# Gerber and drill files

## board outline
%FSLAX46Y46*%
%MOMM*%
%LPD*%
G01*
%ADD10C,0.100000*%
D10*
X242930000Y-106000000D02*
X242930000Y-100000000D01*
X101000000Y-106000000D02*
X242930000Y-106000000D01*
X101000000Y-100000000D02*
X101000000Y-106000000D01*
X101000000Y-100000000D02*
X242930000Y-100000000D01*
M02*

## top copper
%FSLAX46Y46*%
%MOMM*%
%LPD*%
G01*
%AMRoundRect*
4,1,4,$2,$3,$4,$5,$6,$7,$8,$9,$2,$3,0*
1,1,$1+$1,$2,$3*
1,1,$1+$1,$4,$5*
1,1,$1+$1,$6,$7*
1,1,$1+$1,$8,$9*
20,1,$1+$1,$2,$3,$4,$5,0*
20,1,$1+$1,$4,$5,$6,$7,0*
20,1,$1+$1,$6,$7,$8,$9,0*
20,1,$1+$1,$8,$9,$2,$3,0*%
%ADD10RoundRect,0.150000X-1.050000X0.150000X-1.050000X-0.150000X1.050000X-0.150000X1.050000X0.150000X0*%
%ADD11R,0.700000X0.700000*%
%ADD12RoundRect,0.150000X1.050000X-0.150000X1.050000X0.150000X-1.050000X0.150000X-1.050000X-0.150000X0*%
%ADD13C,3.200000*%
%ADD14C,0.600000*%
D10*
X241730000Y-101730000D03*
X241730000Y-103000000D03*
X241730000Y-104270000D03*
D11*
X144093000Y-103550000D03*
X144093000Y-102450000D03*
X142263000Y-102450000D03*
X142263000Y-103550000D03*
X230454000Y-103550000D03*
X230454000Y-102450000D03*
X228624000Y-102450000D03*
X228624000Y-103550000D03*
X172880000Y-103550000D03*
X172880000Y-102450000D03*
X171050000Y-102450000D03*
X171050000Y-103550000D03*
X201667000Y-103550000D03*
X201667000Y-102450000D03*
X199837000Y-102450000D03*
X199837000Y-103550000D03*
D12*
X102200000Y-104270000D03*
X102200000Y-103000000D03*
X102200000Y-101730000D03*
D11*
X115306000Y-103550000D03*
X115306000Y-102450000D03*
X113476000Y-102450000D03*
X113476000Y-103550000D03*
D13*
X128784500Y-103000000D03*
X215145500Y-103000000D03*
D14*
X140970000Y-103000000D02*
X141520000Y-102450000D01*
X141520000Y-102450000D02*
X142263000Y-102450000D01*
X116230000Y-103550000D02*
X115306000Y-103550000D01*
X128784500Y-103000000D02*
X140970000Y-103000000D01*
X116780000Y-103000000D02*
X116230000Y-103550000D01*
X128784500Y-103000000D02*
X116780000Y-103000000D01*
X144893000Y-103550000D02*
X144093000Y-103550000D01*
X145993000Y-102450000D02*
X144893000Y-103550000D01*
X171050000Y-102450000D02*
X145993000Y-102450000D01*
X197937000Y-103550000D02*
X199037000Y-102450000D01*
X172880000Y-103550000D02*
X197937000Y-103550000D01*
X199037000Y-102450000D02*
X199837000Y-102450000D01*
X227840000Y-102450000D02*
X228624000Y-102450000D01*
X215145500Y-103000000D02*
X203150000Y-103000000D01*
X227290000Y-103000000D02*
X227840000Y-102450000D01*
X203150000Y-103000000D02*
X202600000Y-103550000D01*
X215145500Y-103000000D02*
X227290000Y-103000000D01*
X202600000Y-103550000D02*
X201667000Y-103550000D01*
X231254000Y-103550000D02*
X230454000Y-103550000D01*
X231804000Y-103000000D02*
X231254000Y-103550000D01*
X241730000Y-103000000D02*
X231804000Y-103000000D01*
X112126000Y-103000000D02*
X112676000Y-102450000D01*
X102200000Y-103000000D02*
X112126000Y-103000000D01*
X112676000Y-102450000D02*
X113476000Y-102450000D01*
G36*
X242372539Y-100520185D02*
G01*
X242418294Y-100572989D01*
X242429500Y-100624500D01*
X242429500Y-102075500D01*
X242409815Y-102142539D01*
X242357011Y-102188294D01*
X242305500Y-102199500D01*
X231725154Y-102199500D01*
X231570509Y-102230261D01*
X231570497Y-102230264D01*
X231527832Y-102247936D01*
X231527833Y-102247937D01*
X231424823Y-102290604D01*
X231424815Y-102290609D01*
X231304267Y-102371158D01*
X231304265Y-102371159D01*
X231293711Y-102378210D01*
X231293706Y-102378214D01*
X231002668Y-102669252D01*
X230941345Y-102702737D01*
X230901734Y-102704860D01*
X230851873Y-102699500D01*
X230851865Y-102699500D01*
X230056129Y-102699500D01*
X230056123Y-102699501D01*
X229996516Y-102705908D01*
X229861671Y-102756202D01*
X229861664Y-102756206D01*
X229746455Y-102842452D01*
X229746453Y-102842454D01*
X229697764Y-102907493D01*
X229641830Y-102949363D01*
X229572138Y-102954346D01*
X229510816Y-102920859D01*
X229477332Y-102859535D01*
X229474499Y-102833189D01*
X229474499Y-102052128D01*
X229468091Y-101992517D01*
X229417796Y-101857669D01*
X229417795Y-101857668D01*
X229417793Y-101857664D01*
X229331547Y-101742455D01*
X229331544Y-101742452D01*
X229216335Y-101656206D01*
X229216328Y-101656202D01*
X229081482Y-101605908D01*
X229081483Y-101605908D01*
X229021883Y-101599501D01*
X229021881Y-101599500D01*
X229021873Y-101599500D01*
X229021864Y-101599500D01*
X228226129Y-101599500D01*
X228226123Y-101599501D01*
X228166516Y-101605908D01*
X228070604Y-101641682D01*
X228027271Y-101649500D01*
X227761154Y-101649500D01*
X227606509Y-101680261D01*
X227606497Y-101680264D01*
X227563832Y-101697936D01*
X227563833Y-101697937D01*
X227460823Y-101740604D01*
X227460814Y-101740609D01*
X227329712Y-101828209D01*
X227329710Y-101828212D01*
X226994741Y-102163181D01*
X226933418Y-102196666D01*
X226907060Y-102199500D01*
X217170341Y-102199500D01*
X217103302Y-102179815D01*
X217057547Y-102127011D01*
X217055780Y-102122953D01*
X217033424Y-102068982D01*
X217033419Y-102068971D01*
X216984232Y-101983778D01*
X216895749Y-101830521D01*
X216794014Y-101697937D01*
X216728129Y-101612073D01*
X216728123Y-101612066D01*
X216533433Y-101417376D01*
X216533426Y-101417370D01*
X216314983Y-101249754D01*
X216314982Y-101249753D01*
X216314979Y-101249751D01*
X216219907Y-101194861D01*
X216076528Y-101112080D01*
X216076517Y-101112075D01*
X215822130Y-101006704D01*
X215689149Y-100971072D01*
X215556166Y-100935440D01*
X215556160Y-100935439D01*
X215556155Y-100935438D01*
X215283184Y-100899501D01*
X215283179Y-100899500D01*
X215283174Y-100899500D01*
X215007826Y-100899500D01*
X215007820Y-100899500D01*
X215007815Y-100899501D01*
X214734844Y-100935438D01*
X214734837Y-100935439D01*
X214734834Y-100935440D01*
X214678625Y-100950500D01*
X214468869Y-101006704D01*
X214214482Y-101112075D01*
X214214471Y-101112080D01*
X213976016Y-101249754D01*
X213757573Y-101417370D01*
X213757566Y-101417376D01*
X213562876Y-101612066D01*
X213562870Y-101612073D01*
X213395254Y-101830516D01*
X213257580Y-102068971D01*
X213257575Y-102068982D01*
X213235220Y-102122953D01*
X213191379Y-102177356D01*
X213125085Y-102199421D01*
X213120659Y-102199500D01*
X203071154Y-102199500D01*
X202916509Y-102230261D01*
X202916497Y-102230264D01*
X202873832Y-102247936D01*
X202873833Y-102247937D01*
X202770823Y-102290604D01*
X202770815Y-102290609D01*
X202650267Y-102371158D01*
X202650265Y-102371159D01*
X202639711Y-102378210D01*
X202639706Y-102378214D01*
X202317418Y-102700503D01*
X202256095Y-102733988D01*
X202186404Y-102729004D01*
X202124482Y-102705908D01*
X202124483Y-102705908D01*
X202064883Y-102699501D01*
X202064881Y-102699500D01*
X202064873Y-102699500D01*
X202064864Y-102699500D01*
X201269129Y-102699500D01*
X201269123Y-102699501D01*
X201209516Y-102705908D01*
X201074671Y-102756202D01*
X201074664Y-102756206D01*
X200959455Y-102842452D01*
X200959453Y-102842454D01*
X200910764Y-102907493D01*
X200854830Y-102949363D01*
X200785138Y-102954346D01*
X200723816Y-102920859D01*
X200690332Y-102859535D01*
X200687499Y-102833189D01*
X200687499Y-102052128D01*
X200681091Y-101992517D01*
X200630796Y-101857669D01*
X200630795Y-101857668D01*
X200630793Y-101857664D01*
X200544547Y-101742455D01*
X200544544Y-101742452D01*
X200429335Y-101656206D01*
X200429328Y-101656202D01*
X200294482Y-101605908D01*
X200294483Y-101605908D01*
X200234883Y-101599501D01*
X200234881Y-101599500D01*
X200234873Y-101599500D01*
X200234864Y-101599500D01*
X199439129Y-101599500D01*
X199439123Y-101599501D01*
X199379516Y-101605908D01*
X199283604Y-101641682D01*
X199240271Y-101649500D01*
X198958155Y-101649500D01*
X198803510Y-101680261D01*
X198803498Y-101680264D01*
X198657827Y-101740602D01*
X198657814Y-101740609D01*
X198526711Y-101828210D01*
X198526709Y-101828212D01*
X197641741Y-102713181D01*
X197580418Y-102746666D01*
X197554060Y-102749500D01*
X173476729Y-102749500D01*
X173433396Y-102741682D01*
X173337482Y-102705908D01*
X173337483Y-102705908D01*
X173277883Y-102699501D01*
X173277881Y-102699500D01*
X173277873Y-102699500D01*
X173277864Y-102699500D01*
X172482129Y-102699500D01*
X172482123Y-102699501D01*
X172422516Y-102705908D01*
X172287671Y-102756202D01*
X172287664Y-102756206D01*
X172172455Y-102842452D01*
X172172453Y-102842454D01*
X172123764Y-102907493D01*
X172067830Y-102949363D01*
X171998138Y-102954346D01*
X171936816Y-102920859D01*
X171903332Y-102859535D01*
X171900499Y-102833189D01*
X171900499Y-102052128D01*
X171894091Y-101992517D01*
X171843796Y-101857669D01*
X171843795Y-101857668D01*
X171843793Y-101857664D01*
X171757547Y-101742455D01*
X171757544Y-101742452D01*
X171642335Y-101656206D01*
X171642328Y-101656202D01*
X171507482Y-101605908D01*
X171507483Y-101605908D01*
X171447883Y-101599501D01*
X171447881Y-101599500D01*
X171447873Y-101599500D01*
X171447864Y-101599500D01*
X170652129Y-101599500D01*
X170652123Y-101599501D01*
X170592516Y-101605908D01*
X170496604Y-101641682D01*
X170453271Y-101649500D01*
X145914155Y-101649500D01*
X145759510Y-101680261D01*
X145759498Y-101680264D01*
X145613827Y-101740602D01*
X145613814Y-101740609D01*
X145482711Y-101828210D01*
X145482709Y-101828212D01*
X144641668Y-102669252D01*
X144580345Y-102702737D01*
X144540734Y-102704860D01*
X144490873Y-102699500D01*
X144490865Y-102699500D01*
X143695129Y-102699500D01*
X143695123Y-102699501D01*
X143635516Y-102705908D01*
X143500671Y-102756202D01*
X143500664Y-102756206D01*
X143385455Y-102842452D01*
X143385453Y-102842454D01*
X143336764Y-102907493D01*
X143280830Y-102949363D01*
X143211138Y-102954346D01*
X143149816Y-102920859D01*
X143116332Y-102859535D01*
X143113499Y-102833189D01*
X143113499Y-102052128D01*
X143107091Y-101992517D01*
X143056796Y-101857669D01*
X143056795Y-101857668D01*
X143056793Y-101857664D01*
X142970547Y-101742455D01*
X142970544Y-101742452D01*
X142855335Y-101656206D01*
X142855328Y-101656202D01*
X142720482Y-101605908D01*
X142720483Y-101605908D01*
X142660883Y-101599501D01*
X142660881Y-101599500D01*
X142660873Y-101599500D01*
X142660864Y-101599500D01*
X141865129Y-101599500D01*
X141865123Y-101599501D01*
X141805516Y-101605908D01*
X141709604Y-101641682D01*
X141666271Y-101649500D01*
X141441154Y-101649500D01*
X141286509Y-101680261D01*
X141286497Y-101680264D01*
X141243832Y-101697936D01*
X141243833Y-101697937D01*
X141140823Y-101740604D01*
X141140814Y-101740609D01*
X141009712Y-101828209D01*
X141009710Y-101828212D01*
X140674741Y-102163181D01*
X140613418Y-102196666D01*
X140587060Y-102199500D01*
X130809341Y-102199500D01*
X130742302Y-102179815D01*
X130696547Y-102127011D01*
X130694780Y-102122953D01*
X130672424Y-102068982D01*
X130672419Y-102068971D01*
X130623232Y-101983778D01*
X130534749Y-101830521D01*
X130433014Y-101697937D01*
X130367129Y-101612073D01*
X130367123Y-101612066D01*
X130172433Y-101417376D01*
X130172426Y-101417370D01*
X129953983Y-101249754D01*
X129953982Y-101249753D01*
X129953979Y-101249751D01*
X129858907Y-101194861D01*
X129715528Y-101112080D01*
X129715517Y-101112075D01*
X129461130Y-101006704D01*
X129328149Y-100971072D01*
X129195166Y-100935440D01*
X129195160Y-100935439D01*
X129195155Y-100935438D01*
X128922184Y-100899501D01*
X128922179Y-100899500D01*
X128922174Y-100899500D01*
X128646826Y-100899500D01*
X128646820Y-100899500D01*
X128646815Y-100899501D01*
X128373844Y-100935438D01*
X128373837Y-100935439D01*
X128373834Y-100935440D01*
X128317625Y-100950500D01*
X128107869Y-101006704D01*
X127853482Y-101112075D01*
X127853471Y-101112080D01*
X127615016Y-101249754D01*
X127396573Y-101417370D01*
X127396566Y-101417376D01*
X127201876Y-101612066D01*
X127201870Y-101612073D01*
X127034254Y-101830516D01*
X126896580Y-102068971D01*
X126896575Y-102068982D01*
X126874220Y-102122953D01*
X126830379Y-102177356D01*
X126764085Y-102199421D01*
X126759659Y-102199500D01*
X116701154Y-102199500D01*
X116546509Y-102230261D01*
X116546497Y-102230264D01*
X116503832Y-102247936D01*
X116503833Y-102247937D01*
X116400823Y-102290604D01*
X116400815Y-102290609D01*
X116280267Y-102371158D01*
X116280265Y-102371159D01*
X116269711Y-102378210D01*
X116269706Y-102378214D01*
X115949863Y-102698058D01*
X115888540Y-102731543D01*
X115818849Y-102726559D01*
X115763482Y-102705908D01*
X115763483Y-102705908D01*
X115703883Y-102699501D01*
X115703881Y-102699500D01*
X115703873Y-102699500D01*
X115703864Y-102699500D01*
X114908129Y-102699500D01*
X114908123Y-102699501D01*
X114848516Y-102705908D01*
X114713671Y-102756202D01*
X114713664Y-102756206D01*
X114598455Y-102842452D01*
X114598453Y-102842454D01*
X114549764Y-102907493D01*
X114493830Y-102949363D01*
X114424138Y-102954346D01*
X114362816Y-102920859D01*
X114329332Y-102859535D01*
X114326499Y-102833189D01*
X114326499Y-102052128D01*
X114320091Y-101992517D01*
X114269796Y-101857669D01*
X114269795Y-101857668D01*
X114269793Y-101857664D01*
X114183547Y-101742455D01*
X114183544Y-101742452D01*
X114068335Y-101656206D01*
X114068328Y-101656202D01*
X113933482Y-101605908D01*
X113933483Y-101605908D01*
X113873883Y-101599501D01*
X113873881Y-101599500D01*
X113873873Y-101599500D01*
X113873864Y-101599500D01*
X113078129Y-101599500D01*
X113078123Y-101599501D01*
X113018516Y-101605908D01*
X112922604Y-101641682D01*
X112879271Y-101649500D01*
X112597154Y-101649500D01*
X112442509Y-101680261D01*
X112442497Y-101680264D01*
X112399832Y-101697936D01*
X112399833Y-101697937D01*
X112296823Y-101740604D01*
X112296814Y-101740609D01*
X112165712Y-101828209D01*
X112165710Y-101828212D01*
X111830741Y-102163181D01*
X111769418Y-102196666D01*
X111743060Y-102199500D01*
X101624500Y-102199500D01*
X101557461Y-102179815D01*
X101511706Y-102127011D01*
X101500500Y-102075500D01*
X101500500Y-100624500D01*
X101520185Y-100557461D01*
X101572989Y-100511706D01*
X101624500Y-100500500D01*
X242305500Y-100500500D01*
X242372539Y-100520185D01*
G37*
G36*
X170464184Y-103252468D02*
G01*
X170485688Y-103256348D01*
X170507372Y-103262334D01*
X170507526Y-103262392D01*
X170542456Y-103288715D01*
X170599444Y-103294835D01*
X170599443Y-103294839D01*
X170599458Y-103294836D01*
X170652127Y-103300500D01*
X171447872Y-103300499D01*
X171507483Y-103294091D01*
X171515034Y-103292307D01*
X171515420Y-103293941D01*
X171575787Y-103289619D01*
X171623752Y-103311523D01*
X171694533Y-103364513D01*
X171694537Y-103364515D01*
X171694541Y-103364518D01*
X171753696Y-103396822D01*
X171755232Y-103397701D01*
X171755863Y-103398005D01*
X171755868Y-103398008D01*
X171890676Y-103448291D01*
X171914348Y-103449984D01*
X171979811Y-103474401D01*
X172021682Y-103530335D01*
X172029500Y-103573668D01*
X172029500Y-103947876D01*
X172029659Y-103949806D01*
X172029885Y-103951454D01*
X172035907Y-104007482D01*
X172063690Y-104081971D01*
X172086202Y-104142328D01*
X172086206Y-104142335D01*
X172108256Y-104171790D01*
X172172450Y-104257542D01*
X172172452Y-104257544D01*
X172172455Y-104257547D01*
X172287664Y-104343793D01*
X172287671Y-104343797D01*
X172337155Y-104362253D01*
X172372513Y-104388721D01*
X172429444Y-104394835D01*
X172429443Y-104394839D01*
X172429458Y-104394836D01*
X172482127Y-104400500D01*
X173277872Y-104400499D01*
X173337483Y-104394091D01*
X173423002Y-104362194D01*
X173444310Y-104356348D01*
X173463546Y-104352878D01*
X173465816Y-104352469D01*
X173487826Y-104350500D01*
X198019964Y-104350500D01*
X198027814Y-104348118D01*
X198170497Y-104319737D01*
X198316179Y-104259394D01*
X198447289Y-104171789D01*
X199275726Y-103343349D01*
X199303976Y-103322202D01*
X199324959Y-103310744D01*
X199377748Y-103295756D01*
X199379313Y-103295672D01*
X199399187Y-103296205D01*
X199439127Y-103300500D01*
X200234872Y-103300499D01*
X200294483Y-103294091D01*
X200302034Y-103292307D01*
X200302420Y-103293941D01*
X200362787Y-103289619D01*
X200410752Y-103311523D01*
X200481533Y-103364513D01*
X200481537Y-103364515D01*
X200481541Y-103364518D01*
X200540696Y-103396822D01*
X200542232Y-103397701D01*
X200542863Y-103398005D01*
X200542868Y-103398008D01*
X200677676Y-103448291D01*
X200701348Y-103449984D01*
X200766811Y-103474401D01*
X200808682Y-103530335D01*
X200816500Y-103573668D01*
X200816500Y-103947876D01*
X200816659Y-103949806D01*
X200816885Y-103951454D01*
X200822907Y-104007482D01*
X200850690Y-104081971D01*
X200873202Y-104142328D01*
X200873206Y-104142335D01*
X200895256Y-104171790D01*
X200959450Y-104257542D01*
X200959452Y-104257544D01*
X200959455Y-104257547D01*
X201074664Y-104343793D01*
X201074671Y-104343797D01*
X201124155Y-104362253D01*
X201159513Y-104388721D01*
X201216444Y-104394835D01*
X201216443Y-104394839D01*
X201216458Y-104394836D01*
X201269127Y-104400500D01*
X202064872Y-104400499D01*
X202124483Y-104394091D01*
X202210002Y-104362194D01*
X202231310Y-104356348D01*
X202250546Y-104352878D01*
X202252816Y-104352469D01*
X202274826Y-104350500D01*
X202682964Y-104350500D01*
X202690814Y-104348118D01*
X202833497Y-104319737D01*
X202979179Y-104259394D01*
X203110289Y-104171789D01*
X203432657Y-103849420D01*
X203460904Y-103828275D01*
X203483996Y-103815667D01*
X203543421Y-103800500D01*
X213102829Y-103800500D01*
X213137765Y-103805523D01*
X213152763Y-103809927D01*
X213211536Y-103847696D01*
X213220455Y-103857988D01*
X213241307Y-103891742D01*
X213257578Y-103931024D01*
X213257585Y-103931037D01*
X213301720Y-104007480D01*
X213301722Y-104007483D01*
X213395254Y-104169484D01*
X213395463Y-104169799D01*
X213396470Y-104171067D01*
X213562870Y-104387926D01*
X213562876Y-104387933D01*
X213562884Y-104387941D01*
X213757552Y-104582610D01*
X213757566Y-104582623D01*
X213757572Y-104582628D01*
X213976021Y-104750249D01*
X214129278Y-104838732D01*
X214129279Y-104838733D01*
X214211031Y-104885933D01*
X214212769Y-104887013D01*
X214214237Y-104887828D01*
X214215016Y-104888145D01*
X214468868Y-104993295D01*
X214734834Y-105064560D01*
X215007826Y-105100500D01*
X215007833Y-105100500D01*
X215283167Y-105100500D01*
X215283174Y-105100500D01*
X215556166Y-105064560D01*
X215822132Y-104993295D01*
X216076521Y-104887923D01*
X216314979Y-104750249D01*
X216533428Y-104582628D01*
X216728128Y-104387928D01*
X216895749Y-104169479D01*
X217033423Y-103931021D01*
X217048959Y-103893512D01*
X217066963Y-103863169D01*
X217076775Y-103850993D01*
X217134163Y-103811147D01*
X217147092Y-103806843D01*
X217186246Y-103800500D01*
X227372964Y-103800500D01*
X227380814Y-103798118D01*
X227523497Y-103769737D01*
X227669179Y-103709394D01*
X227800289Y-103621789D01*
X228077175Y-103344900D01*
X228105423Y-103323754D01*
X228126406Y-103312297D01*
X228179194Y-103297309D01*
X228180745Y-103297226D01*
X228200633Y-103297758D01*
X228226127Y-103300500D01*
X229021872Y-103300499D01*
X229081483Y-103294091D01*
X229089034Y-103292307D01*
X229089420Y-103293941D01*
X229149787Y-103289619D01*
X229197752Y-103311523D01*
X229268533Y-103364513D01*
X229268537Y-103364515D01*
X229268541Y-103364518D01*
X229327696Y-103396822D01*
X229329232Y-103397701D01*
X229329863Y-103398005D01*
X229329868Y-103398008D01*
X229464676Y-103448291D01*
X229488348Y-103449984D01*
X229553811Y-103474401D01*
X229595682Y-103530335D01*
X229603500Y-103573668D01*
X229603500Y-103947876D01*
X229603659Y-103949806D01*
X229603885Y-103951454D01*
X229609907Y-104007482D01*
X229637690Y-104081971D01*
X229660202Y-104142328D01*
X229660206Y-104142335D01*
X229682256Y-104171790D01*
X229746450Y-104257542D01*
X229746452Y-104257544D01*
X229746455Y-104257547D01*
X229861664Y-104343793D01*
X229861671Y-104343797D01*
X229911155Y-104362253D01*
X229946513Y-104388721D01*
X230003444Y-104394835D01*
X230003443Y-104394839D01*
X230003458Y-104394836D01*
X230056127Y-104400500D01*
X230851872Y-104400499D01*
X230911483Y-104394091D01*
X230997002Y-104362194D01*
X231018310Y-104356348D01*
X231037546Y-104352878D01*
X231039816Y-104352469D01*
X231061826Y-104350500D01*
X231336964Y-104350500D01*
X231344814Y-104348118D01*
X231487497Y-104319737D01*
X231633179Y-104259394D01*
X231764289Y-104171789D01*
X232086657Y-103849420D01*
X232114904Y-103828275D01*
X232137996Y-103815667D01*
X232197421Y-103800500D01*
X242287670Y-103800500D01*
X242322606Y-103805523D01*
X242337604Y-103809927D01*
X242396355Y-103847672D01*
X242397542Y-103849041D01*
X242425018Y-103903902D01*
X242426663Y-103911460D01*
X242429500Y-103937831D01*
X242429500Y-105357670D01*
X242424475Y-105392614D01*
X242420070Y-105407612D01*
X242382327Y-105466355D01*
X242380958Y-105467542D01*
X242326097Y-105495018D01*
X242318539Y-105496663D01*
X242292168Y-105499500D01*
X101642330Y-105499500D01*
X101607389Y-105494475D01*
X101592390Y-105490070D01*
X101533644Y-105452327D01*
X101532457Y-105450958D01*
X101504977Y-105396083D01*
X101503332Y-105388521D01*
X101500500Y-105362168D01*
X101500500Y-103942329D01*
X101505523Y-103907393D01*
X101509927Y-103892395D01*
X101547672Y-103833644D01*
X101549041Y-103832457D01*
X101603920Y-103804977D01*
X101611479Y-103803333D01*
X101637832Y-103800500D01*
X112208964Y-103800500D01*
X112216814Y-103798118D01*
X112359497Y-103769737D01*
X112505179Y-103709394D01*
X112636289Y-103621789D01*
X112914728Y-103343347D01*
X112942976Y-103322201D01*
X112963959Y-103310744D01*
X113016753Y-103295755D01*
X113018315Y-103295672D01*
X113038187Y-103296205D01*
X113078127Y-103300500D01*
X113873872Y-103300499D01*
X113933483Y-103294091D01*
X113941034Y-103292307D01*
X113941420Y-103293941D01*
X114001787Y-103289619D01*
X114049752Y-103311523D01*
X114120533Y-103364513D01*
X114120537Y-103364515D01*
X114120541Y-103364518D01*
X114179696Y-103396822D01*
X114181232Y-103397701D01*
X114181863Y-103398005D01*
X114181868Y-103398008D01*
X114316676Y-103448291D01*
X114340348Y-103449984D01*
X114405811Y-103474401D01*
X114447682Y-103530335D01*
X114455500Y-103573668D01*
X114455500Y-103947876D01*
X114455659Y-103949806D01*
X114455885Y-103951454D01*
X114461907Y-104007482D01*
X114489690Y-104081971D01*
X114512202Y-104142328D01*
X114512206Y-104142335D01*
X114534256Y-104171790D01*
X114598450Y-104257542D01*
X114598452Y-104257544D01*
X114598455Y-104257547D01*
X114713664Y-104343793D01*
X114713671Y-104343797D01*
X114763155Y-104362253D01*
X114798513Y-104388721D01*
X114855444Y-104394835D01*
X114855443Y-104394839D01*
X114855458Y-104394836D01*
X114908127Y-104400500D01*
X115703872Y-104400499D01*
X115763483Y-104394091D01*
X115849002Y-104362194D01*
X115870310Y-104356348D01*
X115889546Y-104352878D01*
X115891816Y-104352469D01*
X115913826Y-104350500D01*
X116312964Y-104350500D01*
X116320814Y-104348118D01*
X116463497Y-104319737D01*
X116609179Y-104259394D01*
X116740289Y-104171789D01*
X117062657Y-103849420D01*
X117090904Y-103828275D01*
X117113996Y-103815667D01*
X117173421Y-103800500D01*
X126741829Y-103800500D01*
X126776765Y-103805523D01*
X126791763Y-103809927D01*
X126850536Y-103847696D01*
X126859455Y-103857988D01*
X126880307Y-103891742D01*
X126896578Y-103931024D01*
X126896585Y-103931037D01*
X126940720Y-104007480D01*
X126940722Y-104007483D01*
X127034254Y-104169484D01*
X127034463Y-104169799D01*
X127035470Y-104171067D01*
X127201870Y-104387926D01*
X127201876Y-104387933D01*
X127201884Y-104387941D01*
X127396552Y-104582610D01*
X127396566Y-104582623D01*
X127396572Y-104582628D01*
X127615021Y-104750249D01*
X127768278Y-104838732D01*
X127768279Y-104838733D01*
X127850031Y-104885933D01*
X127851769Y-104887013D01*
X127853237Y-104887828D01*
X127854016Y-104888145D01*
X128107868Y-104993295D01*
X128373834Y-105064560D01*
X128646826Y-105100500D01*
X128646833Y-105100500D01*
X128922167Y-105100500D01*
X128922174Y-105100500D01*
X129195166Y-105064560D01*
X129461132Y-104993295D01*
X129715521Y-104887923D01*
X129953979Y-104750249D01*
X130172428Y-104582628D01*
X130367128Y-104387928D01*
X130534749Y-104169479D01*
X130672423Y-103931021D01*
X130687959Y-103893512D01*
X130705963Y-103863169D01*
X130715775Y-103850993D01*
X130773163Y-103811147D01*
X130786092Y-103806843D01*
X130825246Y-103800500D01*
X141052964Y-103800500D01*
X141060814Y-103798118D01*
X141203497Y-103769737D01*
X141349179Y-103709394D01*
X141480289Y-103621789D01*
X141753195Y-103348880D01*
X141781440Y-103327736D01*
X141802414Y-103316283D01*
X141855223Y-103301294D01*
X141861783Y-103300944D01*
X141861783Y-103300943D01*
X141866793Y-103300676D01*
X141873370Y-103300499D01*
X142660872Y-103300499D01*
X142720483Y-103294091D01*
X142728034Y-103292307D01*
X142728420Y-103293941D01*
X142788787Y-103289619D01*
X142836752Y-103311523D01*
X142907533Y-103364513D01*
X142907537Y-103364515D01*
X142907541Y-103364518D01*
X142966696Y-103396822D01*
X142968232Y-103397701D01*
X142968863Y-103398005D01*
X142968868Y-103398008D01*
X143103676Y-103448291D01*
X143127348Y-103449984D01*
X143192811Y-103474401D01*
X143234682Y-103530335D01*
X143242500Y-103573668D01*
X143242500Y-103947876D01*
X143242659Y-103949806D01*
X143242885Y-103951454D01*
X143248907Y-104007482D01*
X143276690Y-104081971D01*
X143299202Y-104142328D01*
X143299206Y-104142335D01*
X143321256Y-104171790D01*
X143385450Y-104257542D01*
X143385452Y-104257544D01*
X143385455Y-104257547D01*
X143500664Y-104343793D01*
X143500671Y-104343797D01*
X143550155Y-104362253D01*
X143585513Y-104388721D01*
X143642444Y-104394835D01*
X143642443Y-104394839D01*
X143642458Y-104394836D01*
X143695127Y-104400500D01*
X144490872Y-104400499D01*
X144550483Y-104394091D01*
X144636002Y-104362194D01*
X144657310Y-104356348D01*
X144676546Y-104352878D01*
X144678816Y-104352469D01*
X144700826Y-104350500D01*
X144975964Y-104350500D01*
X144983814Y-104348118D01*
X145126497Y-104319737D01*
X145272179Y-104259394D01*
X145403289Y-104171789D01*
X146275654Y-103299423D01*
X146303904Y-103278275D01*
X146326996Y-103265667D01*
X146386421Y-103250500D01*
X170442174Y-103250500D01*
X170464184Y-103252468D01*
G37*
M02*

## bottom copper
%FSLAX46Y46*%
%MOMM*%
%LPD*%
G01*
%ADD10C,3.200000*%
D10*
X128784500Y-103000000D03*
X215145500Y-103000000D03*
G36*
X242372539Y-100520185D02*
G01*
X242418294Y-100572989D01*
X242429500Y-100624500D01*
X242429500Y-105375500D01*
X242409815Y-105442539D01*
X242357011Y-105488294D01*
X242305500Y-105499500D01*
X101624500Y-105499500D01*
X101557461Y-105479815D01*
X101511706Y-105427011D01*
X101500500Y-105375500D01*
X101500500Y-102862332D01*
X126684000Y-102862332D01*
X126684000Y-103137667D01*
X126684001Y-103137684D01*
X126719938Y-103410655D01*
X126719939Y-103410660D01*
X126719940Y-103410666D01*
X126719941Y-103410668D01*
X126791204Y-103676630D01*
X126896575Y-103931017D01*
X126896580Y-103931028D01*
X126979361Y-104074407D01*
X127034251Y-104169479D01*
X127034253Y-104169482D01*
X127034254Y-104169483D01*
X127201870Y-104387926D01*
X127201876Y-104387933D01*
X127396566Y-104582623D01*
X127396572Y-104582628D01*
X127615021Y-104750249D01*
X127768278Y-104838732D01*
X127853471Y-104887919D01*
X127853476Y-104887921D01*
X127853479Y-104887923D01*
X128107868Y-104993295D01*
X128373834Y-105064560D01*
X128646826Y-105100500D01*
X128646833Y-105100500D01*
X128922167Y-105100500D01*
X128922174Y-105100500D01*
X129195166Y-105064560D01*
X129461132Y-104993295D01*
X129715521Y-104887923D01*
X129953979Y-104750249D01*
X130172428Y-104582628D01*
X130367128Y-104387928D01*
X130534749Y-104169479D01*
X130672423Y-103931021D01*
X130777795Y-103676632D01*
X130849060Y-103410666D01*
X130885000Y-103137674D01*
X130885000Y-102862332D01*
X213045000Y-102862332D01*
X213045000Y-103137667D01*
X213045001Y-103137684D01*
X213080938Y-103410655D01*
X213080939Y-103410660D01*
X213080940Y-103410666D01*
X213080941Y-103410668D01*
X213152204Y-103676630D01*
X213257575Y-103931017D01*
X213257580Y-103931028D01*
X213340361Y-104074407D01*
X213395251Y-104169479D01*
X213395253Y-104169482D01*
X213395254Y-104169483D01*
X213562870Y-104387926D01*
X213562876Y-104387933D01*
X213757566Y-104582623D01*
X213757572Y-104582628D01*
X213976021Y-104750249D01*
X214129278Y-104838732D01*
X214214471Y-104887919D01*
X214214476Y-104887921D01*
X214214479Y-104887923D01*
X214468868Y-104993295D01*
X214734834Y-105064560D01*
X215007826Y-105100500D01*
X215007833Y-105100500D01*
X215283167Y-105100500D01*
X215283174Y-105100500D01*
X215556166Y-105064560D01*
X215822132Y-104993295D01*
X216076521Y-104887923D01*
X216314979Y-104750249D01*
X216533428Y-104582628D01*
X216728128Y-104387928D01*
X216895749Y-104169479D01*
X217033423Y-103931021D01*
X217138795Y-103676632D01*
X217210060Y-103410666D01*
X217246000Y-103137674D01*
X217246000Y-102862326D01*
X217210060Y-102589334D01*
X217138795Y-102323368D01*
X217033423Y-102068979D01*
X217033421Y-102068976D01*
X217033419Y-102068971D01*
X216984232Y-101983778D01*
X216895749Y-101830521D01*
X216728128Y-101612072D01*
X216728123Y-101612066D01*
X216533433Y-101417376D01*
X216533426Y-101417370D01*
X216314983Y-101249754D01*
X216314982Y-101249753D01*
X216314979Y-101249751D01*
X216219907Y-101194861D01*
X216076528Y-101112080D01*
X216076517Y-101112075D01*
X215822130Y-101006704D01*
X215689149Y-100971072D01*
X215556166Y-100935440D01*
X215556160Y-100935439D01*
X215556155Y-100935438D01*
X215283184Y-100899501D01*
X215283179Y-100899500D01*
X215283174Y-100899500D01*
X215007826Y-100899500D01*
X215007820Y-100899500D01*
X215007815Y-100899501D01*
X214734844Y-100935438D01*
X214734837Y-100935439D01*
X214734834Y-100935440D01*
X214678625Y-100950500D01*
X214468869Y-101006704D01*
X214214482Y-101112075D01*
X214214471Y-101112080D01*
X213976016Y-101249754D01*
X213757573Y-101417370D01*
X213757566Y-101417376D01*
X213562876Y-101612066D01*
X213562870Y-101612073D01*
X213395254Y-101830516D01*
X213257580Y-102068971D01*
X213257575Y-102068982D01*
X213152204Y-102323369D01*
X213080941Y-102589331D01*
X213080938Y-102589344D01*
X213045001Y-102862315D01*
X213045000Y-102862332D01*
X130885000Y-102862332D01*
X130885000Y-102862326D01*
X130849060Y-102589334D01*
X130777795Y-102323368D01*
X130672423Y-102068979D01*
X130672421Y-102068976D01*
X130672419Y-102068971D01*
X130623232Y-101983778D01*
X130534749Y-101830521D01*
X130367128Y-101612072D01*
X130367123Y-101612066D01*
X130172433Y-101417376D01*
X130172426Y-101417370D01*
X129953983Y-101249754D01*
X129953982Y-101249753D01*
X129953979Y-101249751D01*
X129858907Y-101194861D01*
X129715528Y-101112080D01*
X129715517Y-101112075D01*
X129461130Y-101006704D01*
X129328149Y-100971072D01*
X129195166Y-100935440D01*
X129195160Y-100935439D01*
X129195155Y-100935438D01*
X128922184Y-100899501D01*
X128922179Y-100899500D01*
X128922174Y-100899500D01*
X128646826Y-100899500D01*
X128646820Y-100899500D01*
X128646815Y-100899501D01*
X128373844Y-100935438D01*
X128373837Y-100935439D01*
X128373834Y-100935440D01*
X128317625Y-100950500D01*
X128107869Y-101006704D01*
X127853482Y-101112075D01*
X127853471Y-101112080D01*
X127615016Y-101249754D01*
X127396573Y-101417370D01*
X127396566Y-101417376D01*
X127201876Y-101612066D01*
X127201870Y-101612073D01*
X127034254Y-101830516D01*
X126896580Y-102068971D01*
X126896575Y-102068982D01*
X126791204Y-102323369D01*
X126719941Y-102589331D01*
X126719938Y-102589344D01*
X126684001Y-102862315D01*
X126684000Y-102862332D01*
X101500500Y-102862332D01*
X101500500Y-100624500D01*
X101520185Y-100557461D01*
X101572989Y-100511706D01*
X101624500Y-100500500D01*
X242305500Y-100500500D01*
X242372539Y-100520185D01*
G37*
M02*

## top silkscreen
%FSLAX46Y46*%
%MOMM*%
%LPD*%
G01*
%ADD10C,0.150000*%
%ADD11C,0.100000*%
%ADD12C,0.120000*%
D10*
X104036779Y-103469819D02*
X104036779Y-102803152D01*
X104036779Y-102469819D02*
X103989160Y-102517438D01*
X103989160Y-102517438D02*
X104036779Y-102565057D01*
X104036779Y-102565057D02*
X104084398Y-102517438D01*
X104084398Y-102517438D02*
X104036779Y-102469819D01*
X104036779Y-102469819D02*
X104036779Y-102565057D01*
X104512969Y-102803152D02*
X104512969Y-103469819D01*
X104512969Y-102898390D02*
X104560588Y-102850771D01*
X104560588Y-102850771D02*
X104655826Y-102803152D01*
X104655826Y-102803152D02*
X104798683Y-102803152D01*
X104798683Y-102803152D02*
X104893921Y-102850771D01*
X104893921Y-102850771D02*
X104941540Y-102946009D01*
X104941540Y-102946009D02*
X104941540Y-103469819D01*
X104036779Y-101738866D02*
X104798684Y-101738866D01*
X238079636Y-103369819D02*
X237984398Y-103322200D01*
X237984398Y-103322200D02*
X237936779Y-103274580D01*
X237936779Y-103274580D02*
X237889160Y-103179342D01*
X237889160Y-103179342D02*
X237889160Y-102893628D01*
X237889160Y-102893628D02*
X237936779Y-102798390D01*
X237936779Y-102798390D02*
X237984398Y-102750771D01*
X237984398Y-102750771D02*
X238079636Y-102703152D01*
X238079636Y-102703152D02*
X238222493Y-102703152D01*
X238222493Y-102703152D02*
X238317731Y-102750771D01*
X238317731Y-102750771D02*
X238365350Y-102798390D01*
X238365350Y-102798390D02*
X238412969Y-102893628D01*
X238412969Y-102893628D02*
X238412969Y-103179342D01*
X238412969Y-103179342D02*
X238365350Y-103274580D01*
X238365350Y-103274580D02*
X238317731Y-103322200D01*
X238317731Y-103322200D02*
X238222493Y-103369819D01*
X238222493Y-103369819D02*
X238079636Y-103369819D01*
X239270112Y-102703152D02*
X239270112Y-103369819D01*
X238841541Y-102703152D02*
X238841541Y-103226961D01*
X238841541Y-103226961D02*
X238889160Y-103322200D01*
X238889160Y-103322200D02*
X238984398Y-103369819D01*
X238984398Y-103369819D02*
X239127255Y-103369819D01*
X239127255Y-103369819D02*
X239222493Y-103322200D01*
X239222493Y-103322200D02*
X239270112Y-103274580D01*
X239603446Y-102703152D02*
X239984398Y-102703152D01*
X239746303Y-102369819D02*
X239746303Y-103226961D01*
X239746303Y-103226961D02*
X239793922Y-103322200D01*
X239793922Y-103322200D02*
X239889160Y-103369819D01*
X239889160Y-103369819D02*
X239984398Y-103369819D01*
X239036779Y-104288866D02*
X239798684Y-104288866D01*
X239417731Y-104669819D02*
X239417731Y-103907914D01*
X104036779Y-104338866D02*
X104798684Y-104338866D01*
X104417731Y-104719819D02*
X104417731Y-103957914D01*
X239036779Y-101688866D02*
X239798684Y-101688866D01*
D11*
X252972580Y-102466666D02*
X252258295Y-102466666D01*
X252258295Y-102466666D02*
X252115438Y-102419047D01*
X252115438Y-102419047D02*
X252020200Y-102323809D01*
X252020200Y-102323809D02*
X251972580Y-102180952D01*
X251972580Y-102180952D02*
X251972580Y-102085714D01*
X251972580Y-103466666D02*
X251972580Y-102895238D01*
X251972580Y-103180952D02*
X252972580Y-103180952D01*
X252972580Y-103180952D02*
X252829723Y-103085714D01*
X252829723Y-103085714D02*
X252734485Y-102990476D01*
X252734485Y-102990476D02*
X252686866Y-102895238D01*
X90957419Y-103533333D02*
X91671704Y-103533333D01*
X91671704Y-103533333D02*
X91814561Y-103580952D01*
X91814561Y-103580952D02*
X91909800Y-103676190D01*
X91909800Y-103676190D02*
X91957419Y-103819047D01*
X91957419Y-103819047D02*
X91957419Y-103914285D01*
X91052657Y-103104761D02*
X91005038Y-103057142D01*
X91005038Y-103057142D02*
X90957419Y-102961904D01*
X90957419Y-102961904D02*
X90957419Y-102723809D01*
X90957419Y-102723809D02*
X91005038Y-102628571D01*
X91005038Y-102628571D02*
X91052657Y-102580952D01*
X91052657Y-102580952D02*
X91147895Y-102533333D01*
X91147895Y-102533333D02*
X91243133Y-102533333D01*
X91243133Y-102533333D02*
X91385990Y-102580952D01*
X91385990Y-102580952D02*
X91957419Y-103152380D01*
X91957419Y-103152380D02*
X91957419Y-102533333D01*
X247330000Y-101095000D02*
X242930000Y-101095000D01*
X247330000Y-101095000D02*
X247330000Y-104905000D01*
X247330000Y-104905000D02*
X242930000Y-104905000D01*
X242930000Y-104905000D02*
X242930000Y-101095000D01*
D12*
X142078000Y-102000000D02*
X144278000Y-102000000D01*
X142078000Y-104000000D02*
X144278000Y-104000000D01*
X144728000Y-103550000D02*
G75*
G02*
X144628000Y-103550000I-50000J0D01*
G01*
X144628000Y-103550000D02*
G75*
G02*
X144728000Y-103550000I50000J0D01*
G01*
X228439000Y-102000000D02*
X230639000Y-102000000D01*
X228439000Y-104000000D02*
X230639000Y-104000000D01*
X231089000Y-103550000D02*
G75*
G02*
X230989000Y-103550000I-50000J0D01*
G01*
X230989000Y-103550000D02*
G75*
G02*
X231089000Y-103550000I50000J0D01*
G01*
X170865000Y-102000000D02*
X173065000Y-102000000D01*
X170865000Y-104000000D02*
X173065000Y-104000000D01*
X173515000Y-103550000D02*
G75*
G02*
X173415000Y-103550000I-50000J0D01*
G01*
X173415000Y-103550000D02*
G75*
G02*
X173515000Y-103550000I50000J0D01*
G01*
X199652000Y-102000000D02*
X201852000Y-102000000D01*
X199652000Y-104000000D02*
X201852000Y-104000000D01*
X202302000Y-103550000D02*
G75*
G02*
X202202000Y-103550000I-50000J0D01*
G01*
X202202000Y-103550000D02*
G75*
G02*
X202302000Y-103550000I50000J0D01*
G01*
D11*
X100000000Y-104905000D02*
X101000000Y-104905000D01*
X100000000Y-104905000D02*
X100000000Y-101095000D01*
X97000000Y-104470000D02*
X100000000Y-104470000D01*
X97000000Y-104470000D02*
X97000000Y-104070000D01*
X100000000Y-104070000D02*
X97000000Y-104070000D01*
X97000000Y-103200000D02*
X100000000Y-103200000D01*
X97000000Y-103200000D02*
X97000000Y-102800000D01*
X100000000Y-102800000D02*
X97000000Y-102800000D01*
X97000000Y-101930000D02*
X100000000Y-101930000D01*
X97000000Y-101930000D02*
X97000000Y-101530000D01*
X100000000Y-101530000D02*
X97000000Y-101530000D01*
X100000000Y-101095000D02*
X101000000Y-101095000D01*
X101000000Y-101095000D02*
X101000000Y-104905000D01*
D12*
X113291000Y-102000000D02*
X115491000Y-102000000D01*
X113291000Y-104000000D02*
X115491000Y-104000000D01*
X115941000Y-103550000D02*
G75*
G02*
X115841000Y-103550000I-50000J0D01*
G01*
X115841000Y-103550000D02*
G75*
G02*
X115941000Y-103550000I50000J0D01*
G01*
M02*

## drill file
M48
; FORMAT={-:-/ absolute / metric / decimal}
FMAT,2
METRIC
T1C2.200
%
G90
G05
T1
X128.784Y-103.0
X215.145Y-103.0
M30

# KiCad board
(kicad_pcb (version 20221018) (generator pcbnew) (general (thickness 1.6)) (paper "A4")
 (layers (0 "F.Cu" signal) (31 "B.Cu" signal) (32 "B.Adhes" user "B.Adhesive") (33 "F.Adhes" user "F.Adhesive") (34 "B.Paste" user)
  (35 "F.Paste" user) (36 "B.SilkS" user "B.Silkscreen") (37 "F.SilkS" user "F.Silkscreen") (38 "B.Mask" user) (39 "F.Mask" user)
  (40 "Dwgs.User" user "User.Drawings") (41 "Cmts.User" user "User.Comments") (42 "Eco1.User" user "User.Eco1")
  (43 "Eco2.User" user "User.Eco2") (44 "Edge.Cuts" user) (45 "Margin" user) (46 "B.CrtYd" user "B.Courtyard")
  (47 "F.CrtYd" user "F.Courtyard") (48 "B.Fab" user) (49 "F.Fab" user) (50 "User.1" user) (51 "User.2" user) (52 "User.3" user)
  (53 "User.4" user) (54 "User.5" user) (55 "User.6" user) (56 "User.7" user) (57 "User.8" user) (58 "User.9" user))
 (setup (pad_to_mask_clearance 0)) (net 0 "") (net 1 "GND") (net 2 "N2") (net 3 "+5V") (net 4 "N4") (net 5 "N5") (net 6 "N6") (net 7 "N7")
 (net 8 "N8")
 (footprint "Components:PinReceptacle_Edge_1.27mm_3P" (layer "F.Cu") (at 242.93 103 -90)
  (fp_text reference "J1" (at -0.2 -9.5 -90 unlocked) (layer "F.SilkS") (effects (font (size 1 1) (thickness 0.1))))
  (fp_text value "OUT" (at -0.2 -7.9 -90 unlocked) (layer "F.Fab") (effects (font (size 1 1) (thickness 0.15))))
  (fp_line (start -1.905 -4.4) (end -1.905 0) (stroke (width 0.1) (type default)) (layer "F.SilkS"))
  (fp_line (start -1.905 -4.4) (end 1.905 -4.4) (stroke (width 0.1) (type default)) (layer "F.SilkS"))
  (fp_line (start 1.905 -4.4) (end 1.905 0) (stroke (width 0.1) (type default)) (layer "F.SilkS"))
  (fp_line (start 1.905 0) (end -1.905 0) (stroke (width 0.1) (type default)) (layer "F.SilkS"))
  (pad "1" smd roundrect (at -1.27 1.2 270) (size 0.6 2.4) (layers "F.Cu" "F.Paste" "F.Mask") (roundrect_rratio 0.25) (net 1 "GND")
   (thermal_bridge_angle 45))
  (pad "2" smd roundrect (at 0 1.2 270) (size 0.6 2.4) (layers "F.Cu" "F.Paste" "F.Mask") (roundrect_rratio 0.25) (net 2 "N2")
   (thermal_bridge_angle 45))
  (pad "3" smd roundrect (at 1.27 1.2 270) (size 0.6 2.4) (layers "F.Cu" "F.Paste" "F.Mask") (roundrect_rratio 0.25) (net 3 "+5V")
   (thermal_bridge_angle 45)))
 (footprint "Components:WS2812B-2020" (layer "F.Cu") (at 143.178 103)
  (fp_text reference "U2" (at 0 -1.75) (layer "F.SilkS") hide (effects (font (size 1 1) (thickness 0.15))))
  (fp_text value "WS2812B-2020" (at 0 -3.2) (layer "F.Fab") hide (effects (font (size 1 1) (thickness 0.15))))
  (fp_line (start -1.1 -1) (end 1.1 -1) (stroke (width 0.12) (type solid)) (layer "F.SilkS"))
  (fp_line (start -1.1 1) (end 1.1 1) (stroke (width 0.12) (type solid)) (layer "F.SilkS"))
  (fp_circle (center 1.5 0.55) (end 1.45 0.55) (stroke (width 0.12) (type solid)) (fill none) (layer "F.SilkS"))
  (pad "1" smd rect (at 0.915 0.55) (size 0.7 0.7) (layers "F.Cu" "F.Paste" "F.Mask") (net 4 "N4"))
  (pad "2" smd rect (at 0.915 -0.55) (size 0.7 0.7) (layers "F.Cu" "F.Paste" "F.Mask") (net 1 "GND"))
  (pad "3" smd rect (at -0.915 -0.55) (size 0.7 0.7) (layers "F.Cu" "F.Paste" "F.Mask") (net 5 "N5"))
  (pad "4" smd rect (at -0.915 0.55) (size 0.7 0.7) (layers "F.Cu" "F.Paste" "F.Mask") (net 3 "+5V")))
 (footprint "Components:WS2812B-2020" (layer "F.Cu") (at 229.539 103)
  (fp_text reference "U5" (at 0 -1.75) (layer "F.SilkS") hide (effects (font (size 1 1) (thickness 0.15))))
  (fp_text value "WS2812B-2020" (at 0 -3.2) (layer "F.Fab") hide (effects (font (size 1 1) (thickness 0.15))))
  (fp_line (start -1.1 -1) (end 1.1 -1) (stroke (width 0.12) (type solid)) (layer "F.SilkS"))
  (fp_line (start -1.1 1) (end 1.1 1) (stroke (width 0.12) (type solid)) (layer "F.SilkS"))
  (fp_circle (center 1.5 0.55) (end 1.45 0.55) (stroke (width 0.12) (type solid)) (fill none) (layer "F.SilkS"))
  (pad "1" smd rect (at 0.915 0.55) (size 0.7 0.7) (layers "F.Cu" "F.Paste" "F.Mask") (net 2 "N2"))
  (pad "2" smd rect (at 0.915 -0.55) (size 0.7 0.7) (layers "F.Cu" "F.Paste" "F.Mask") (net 1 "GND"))
  (pad "3" smd rect (at -0.915 -0.55) (size 0.7 0.7) (layers "F.Cu" "F.Paste" "F.Mask") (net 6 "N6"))
  (pad "4" smd rect (at -0.915 0.55) (size 0.7 0.7) (layers "F.Cu" "F.Paste" "F.Mask") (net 3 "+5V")))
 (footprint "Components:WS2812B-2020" (layer "F.Cu") (at 171.965 103)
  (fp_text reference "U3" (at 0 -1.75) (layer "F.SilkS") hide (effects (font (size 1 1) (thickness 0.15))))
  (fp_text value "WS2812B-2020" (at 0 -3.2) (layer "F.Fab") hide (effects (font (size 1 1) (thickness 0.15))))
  (fp_line (start -1.1 -1) (end 1.1 -1) (stroke (width 0.12) (type solid)) (layer "F.SilkS"))
  (fp_line (start -1.1 1) (end 1.1 1) (stroke (width 0.12) (type solid)) (layer "F.SilkS"))
  (fp_circle (center 1.5 0.55) (end 1.45 0.55) (stroke (width 0.12) (type solid)) (fill none) (layer "F.SilkS"))
  (pad "1" smd rect (at 0.915 0.55) (size 0.7 0.7) (layers "F.Cu" "F.Paste" "F.Mask") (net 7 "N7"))
  (pad "2" smd rect (at 0.915 -0.55) (size 0.7 0.7) (layers "F.Cu" "F.Paste" "F.Mask") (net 1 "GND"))
  (pad "3" smd rect (at -0.915 -0.55) (size 0.7 0.7) (layers "F.Cu" "F.Paste" "F.Mask") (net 4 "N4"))
  (pad "4" smd rect (at -0.915 0.55) (size 0.7 0.7) (layers "F.Cu" "F.Paste" "F.Mask") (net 3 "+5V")))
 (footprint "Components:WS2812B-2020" (layer "F.Cu") (at 200.752 103)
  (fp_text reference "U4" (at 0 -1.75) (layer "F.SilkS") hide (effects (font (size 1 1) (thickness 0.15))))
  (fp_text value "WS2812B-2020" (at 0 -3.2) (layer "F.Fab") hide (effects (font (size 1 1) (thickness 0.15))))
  (fp_line (start -1.1 -1) (end 1.1 -1) (stroke (width 0.12) (type solid)) (layer "F.SilkS"))
  (fp_line (start -1.1 1) (end 1.1 1) (stroke (width 0.12) (type solid)) (layer "F.SilkS"))
  (fp_circle (center 1.5 0.55) (end 1.45 0.55) (stroke (width 0.12) (type solid)) (fill none) (layer "F.SilkS"))
  (pad "1" smd rect (at 0.915 0.55) (size 0.7 0.7) (layers "F.Cu" "F.Paste" "F.Mask") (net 6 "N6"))
  (pad "2" smd rect (at 0.915 -0.55) (size 0.7 0.7) (layers "F.Cu" "F.Paste" "F.Mask") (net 1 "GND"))
  (pad "3" smd rect (at -0.915 -0.55) (size 0.7 0.7) (layers "F.Cu" "F.Paste" "F.Mask") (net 7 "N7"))
  (pad "4" smd rect (at -0.915 0.55) (size 0.7 0.7) (layers "F.Cu" "F.Paste" "F.Mask") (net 3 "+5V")))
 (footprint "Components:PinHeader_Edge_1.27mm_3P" (layer "F.Cu") (at 101 103 90)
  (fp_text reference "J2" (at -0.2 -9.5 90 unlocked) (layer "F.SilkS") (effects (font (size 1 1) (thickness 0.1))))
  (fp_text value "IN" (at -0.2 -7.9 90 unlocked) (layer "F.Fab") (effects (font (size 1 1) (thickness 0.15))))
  (fp_line (start -1.905 -1) (end -1.905 0) (stroke (width 0.1) (type default)) (layer "F.SilkS"))
  (fp_line (start -1.905 -1) (end 1.905 -1) (stroke (width 0.1) (type default)) (layer "F.SilkS"))
  (fp_line (start -1.47 -4) (end -1.47 -1) (stroke (width 0.1) (type default)) (layer "F.SilkS"))
  (fp_line (start -1.47 -4) (end -1.07 -4) (stroke (width 0.1) (type default)) (layer "F.SilkS"))
  (fp_line (start -1.07 -1) (end -1.07 -4) (stroke (width 0.1) (type default)) (layer "F.SilkS"))
  (fp_line (start -0.2 -4) (end -0.2 -1) (stroke (width 0.1) (type default)) (layer "F.SilkS"))
  (fp_line (start -0.2 -4) (end 0.2 -4) (stroke (width 0.1) (type default)) (layer "F.SilkS"))
  (fp_line (start 0.2 -1) (end 0.2 -4) (stroke (width 0.1) (type default)) (layer "F.SilkS"))
  (fp_line (start 1.07 -4) (end 1.07 -1) (stroke (width 0.1) (type default)) (layer "F.SilkS"))
  (fp_line (start 1.07 -4) (end 1.47 -4) (stroke (width 0.1) (type default)) (layer "F.SilkS"))
  (fp_line (start 1.47 -1) (end 1.47 -4) (stroke (width 0.1) (type default)) (layer "F.SilkS"))
  (fp_line (start 1.905 -1) (end 1.905 0) (stroke (width 0.1) (type default)) (layer "F.SilkS"))
  (fp_line (start 1.905 0) (end -1.905 0) (stroke (width 0.1) (type default)) (layer "F.SilkS"))
  (pad "1" smd roundrect (at -1.27 1.2 90) (size 0.6 2.4) (layers "F.Cu" "F.Paste" "F.Mask") (roundrect_rratio 0.25) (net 3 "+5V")
   (thermal_bridge_angle 45))
  (pad "2" smd roundrect (at 0 1.2 90) (size 0.6 2.4) (layers "F.Cu" "F.Paste" "F.Mask") (roundrect_rratio 0.25) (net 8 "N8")
   (thermal_bridge_angle 45))
  (pad "3" smd roundrect (at 1.27 1.2 90) (size 0.6 2.4) (layers "F.Cu" "F.Paste" "F.Mask") (roundrect_rratio 0.25) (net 1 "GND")
   (thermal_bridge_angle 45)))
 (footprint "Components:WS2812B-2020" (layer "F.Cu") (at 114.391 103)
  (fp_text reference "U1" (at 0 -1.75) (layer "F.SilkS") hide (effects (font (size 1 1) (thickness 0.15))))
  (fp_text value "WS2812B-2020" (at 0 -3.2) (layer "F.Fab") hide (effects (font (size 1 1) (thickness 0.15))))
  (fp_line (start -1.1 -1) (end 1.1 -1) (stroke (width 0.12) (type solid)) (layer "F.SilkS"))
  (fp_line (start -1.1 1) (end 1.1 1) (stroke (width 0.12) (type solid)) (layer "F.SilkS"))
  (fp_circle (center 1.5 0.55) (end 1.45 0.55) (stroke (width 0.12) (type solid)) (fill none) (layer "F.SilkS"))
  (pad "1" smd rect (at 0.915 0.55) (size 0.7 0.7) (layers "F.Cu" "F.Paste" "F.Mask") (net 5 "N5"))
  (pad "2" smd rect (at 0.915 -0.55) (size 0.7 0.7) (layers "F.Cu" "F.Paste" "F.Mask") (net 1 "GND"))
  (pad "3" smd rect (at -0.915 -0.55) (size 0.7 0.7) (layers "F.Cu" "F.Paste" "F.Mask") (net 8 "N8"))
  (pad "4" smd rect (at -0.915 0.55) (size 0.7 0.7) (layers "F.Cu" "F.Paste" "F.Mask") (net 3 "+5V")))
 (gr_line (start 242.93 106) (end 242.93 100) (stroke (width 0.1) (type default)) (layer "Edge.Cuts"))
 (gr_line (start 101 106) (end 242.93 106) (stroke (width 0.1) (type default)) (layer "Edge.Cuts"))
 (gr_line (start 101 100) (end 101 106) (stroke (width 0.1) (type default)) (layer "Edge.Cuts"))
 (gr_line (start 101 100) (end 242.93 100) (stroke (width 0.1) (type default)) (layer "Edge.Cuts"))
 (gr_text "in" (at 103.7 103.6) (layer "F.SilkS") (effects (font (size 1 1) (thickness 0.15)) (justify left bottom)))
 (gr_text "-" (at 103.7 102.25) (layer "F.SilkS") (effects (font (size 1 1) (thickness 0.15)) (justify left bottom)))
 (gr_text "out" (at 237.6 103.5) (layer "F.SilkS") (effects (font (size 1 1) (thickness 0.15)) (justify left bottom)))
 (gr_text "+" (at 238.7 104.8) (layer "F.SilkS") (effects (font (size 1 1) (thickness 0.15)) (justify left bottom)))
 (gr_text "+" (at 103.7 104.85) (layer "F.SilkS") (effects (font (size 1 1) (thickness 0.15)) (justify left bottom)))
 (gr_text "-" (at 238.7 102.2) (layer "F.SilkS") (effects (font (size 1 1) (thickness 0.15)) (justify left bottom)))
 (segment (start 140.97 103) (end 141.52 102.45) (width 0.6) (layer "F.Cu") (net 5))
 (segment (start 141.52 102.45) (end 142.263 102.45) (width 0.6) (layer "F.Cu") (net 5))
 (segment (start 116.23 103.55) (end 115.306 103.55) (width 0.6) (layer "F.Cu") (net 5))
 (segment (start 128.7845 103) (end 140.97 103) (width 0.6) (layer "F.Cu") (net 5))
 (segment (start 116.78 103) (end 116.23 103.55) (width 0.6) (layer "F.Cu") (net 5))
 (segment (start 128.7845 103) (end 116.78 103) (width 0.6) (layer "F.Cu") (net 5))
 (via (at 128.7845 103) (size 3.2) (drill 2.2) (layers "F.Cu" "B.Cu") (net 5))
 (segment (start 144.893 103.55) (end 144.093 103.55) (width 0.6) (layer "F.Cu") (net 4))
 (segment (start 145.993 102.45) (end 144.893 103.55) (width 0.6) (layer "F.Cu") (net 4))
 (segment (start 171.05 102.45) (end 145.993 102.45) (width 0.6) (layer "F.Cu") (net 4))
 (segment (start 197.937 103.55) (end 199.037 102.45) (width 0.6) (layer "F.Cu") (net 7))
 (segment (start 172.88 103.55) (end 197.937 103.55) (width 0.6) (layer "F.Cu") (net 7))
 (segment (start 199.037 102.45) (end 199.837 102.45) (width 0.6) (layer "F.Cu") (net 7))
 (segment (start 227.84 102.45) (end 228.624 102.45) (width 0.6) (layer "F.Cu") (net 6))
 (segment (start 215.1455 103) (end 203.15 103) (width 0.6) (layer "F.Cu") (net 6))
 (segment (start 227.29 103) (end 227.84 102.45) (width 0.6) (layer "F.Cu") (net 6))
 (segment (start 203.15 103) (end 202.6 103.55) (width 0.6) (layer "F.Cu") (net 6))
 (segment (start 215.1455 103) (end 227.29 103) (width 0.6) (layer "F.Cu") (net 6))
 (segment (start 202.6 103.55) (end 201.667 103.55) (width 0.6) (layer "F.Cu") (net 6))
 (via (at 215.1455 103) (size 3.2) (drill 2.2) (layers "F.Cu" "B.Cu") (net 6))
 (segment (start 231.254 103.55) (end 230.454 103.55) (width 0.6) (layer "F.Cu") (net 2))
 (segment (start 231.804 103) (end 231.254 103.55) (width 0.6) (layer "F.Cu") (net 2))
 (segment (start 241.73 103) (end 231.804 103) (width 0.6) (layer "F.Cu") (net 2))
 (segment (start 112.126 103) (end 112.676 102.45) (width 0.6) (layer "F.Cu") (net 8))
 (segment (start 102.2 103) (end 112.126 103) (width 0.6) (layer "F.Cu") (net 8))
 (segment (start 112.676 102.45) (end 113.476 102.45) (width 0.6) (layer "F.Cu") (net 8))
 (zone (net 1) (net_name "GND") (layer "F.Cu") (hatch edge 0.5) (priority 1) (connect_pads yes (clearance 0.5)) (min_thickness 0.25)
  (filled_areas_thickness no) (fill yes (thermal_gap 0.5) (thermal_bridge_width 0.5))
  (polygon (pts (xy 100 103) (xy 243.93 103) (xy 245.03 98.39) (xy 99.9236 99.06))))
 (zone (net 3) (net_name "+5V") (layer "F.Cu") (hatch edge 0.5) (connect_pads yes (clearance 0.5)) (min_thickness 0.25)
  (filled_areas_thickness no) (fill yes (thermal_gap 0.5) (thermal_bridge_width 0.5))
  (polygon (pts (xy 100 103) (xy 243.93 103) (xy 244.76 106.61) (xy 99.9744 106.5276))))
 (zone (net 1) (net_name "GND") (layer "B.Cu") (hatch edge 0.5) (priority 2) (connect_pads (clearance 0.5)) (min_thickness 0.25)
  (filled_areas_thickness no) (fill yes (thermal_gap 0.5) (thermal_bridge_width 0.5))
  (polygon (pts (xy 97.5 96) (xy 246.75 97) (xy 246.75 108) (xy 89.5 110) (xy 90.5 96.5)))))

